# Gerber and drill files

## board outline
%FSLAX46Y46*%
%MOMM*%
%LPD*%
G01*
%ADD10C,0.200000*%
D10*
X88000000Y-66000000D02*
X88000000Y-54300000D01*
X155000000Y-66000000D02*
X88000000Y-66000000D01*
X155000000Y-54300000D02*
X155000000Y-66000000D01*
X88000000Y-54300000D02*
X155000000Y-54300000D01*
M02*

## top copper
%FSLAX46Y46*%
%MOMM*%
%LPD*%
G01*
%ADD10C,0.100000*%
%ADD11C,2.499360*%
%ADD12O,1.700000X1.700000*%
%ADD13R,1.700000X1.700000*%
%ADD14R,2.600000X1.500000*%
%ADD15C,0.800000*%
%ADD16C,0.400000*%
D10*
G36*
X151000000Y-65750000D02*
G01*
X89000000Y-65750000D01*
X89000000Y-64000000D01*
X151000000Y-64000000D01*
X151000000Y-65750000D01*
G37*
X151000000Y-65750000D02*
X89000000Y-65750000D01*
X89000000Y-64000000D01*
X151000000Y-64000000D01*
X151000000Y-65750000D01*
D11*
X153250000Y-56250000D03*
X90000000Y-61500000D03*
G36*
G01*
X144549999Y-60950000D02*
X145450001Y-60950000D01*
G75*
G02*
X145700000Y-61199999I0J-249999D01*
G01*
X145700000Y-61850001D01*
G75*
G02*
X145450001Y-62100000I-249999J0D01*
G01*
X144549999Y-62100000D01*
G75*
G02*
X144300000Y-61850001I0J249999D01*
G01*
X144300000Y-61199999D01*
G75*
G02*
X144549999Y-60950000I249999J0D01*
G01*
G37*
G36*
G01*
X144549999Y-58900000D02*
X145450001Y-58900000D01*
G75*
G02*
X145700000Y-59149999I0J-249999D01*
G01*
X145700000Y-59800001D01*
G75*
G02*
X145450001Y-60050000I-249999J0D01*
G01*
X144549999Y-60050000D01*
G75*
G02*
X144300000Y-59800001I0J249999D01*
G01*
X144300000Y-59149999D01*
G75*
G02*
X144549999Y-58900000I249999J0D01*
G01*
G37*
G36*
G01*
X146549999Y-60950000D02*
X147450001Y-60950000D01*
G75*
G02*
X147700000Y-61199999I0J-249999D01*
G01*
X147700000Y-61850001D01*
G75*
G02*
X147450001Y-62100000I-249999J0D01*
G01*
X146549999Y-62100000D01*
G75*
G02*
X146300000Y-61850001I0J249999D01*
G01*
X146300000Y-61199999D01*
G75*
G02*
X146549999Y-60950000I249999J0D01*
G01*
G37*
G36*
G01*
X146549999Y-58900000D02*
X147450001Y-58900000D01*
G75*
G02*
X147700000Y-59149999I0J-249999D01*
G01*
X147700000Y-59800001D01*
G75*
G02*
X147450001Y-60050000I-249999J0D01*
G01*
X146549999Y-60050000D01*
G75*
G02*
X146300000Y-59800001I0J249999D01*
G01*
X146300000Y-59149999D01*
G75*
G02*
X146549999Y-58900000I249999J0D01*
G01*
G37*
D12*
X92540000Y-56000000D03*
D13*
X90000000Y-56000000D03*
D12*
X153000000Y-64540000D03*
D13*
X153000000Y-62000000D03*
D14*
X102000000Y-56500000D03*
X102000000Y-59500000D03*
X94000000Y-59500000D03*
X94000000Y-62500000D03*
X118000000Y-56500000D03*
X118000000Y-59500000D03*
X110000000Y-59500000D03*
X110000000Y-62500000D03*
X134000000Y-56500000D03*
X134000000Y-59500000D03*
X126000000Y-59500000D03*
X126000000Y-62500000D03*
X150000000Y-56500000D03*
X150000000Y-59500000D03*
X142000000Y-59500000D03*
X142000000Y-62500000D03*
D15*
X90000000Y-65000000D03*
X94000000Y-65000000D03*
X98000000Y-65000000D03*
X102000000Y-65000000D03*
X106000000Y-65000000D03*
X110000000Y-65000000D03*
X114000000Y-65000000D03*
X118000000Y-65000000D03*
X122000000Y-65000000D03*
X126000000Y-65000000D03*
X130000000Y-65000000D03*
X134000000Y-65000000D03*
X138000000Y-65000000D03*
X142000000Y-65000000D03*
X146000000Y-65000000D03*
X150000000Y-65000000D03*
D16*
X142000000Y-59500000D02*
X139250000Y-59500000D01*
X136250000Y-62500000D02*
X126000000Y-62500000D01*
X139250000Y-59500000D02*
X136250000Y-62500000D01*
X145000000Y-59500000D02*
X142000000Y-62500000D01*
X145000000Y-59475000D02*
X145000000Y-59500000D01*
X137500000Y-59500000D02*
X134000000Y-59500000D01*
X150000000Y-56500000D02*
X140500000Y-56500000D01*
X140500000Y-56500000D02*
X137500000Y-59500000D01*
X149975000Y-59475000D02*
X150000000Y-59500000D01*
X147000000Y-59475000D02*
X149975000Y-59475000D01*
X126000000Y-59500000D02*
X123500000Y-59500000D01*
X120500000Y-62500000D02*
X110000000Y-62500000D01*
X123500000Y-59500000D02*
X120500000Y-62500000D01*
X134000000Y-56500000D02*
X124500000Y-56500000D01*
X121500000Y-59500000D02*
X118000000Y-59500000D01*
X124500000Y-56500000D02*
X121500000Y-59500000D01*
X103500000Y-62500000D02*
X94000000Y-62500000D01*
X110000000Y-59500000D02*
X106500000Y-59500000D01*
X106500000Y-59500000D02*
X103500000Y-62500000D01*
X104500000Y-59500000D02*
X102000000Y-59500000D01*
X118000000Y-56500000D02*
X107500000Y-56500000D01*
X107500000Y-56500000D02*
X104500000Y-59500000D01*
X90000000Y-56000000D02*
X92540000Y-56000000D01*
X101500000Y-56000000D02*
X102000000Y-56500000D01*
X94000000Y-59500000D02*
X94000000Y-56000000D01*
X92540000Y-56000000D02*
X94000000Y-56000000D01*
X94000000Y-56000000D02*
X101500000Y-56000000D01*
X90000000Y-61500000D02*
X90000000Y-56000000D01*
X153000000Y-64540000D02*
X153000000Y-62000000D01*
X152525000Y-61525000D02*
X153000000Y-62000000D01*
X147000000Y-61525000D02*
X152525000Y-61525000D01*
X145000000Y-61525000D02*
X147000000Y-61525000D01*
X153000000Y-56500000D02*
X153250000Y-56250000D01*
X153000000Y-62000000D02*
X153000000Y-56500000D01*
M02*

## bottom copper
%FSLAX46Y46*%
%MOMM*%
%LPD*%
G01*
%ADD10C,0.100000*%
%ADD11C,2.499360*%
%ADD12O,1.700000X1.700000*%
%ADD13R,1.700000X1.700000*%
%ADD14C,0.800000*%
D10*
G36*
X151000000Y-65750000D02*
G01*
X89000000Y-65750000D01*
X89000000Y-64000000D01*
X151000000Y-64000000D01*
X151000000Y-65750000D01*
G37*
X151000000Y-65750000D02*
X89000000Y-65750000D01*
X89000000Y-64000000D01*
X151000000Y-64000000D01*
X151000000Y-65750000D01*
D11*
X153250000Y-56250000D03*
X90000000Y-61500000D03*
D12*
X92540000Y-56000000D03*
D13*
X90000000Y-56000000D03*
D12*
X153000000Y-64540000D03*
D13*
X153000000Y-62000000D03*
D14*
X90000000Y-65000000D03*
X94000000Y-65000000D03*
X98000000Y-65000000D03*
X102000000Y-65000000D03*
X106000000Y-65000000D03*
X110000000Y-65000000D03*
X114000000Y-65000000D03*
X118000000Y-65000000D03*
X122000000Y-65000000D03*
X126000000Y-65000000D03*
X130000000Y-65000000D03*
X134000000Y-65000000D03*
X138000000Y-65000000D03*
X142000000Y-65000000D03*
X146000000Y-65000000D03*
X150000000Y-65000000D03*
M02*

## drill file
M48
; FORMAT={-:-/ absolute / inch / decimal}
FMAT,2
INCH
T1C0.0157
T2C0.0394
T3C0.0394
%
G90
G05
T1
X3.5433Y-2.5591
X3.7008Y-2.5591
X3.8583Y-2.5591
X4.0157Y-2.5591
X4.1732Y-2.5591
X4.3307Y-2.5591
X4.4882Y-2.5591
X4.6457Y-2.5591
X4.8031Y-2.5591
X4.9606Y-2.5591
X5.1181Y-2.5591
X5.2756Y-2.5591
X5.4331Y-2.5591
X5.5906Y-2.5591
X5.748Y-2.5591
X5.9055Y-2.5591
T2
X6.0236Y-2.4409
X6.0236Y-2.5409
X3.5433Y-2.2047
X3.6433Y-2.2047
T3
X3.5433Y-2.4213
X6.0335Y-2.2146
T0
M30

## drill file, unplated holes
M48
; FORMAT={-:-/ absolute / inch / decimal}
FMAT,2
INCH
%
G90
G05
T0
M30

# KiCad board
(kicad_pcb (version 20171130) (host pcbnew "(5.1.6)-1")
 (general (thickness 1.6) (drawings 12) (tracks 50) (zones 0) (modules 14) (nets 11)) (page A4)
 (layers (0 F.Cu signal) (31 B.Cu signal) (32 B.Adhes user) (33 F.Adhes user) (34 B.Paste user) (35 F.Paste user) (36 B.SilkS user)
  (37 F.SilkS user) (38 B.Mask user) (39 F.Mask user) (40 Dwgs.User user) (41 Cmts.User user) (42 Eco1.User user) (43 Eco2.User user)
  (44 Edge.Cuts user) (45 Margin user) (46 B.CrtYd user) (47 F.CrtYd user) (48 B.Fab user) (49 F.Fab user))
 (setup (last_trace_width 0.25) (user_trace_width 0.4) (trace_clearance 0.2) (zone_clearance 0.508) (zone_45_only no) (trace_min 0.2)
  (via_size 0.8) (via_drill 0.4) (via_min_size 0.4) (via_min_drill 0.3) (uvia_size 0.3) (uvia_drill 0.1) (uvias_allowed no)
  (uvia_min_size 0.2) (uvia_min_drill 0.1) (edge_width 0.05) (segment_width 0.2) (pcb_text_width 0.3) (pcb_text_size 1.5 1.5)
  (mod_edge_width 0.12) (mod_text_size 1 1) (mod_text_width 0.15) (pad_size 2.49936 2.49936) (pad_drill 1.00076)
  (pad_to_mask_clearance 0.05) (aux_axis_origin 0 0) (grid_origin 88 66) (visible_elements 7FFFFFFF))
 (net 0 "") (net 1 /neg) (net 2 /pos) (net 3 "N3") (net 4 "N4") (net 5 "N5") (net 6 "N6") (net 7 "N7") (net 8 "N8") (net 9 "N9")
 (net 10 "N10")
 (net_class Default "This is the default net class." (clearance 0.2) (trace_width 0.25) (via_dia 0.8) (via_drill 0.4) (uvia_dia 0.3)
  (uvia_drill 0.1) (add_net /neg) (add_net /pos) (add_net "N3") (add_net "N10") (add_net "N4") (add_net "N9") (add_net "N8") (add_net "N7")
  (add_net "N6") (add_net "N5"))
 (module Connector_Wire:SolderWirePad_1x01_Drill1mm (layer F.Cu) (at 153.25 56.25)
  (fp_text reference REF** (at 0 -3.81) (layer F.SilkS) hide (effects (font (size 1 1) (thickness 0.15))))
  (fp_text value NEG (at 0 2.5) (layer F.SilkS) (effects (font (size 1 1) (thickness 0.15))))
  (pad 1 thru_hole circle (at 0 0) (size 2.49936 2.49936) (drill 1.00076) (layers *.Cu *.Mask) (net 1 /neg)))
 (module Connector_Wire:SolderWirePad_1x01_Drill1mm (layer F.Cu) (at 90 61.5)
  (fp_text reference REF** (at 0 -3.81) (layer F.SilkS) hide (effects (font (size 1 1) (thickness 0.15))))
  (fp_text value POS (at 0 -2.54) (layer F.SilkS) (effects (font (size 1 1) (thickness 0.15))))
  (pad 1 thru_hole circle (at 0 0) (size 2.49936 2.49936) (drill 1.00076) (layers *.Cu *.Mask) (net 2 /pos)))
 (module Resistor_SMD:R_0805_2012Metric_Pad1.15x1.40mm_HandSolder (layer F.Cu) (at 145 60.5 270)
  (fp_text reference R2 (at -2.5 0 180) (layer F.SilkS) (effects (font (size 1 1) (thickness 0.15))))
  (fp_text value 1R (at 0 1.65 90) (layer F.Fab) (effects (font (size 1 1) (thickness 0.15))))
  (pad 2 smd roundrect (at 1.025 0 270) (size 1.15 1.4) (layers F.Cu F.Paste F.Mask) (roundrect_rratio 0.217391) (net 1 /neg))
  (pad 1 smd roundrect (at -1.025 0 270) (size 1.15 1.4) (layers F.Cu F.Paste F.Mask) (roundrect_rratio 0.217391) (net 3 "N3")))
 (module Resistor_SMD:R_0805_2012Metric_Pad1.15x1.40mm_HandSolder (layer F.Cu) (at 147 60.5 270)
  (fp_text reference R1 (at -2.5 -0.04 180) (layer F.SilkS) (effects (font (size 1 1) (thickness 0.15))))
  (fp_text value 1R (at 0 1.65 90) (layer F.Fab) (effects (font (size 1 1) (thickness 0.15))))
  (pad 2 smd roundrect (at 1.025 0 270) (size 1.15 1.4) (layers F.Cu F.Paste F.Mask) (roundrect_rratio 0.217391) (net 1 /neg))
  (pad 1 smd roundrect (at -1.025 0 270) (size 1.15 1.4) (layers F.Cu F.Paste F.Mask) (roundrect_rratio 0.217391) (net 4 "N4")))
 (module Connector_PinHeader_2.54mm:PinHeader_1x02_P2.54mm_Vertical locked (layer B.Cu) (at 90 56 270)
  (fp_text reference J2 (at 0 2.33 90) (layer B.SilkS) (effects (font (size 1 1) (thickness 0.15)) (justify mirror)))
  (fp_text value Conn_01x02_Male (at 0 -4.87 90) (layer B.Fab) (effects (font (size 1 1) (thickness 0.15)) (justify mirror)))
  (pad 2 thru_hole oval (at 0 -2.54 270) (size 1.7 1.7) (drill 1) (layers *.Cu *.Mask) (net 2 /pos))
  (pad 1 thru_hole rect (at 0 0 270) (size 1.7 1.7) (drill 1) (layers *.Cu *.Mask) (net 2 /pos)))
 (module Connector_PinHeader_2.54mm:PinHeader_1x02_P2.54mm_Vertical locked (layer B.Cu) (at 153 62 180)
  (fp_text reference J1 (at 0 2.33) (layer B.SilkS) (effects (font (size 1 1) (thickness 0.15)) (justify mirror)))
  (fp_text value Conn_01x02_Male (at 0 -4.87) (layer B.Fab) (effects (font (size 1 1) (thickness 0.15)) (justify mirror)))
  (pad 2 thru_hole oval (at 0 -2.54 180) (size 1.7 1.7) (drill 1) (layers *.Cu *.Mask) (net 1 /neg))
  (pad 1 thru_hole rect (at 0 0 180) (size 1.7 1.7) (drill 1) (layers *.Cu *.Mask) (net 1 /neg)))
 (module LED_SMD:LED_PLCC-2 (layer F.Cu) (at 102 58 90)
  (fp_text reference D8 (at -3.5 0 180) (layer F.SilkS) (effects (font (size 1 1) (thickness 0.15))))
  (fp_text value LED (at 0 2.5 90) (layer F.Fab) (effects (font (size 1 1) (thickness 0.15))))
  (pad 2 smd rect (at 1.5 0 90) (size 1.5 2.6) (layers F.Cu F.Paste F.Mask) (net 2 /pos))
  (pad 1 smd rect (at -1.5 0 90) (size 1.5 2.6) (layers F.Cu F.Paste F.Mask) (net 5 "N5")))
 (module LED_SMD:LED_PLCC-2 (layer F.Cu) (at 94 61 90)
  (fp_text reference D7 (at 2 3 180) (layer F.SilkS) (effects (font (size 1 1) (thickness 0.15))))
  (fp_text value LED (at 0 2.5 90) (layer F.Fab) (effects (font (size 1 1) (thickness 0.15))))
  (pad 2 smd rect (at 1.5 0 90) (size 1.5 2.6) (layers F.Cu F.Paste F.Mask) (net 2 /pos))
  (pad 1 smd rect (at -1.5 0 90) (size 1.5 2.6) (layers F.Cu F.Paste F.Mask) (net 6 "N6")))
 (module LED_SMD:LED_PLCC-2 (layer F.Cu) (at 118 58 90)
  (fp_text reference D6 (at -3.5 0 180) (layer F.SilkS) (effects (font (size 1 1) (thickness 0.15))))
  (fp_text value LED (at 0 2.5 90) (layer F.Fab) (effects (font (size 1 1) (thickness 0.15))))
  (pad 2 smd rect (at 1.5 0 90) (size 1.5 2.6) (layers F.Cu F.Paste F.Mask) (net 5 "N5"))
  (pad 1 smd rect (at -1.5 0 90) (size 1.5 2.6) (layers F.Cu F.Paste F.Mask) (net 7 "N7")))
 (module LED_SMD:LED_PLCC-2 (layer F.Cu) (at 110 61 90)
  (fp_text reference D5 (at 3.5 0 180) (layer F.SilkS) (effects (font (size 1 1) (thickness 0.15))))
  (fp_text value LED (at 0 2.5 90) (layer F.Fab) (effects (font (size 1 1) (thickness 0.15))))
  (pad 2 smd rect (at 1.5 0 90) (size 1.5 2.6) (layers F.Cu F.Paste F.Mask) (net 6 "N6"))
  (pad 1 smd rect (at -1.5 0 90) (size 1.5 2.6) (layers F.Cu F.Paste F.Mask) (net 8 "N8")))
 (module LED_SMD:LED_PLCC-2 (layer F.Cu) (at 134 58 90)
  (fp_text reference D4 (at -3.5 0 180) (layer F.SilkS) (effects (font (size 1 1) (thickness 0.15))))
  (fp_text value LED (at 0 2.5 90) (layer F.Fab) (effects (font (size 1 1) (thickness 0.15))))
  (pad 2 smd rect (at 1.5 0 90) (size 1.5 2.6) (layers F.Cu F.Paste F.Mask) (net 7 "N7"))
  (pad 1 smd rect (at -1.5 0 90) (size 1.5 2.6) (layers F.Cu F.Paste F.Mask) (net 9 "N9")))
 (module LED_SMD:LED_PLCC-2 (layer F.Cu) (at 126 61 90)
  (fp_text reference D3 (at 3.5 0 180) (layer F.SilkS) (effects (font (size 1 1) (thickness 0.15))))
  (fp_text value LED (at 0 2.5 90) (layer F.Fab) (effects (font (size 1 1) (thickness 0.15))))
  (pad 2 smd rect (at 1.5 0 90) (size 1.5 2.6) (layers F.Cu F.Paste F.Mask) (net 8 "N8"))
  (pad 1 smd rect (at -1.5 0 90) (size 1.5 2.6) (layers F.Cu F.Paste F.Mask) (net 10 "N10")))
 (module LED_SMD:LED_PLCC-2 (layer F.Cu) (at 150 58 90)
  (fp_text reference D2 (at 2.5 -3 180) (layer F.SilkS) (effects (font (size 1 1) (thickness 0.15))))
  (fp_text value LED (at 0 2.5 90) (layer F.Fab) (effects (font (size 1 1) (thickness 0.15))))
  (pad 2 smd rect (at 1.5 0 90) (size 1.5 2.6) (layers F.Cu F.Paste F.Mask) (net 9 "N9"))
  (pad 1 smd rect (at -1.5 0 90) (size 1.5 2.6) (layers F.Cu F.Paste F.Mask) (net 4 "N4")))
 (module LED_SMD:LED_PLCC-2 (layer F.Cu) (at 142 61 90)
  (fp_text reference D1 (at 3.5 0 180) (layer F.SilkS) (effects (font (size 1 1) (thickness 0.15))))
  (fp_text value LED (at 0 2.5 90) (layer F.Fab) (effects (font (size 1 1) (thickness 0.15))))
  (pad 2 smd rect (at 1.5 0 90) (size 1.5 2.6) (layers F.Cu F.Paste F.Mask) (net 10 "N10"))
  (pad 1 smd rect (at -1.5 0 90) (size 1.5 2.6) (layers F.Cu F.Paste F.Mask) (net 3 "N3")))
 (gr_poly (pts (xy 151 65.75) (xy 89 65.75) (xy 89 64) (xy 151 64)) (layer B.Cu) (width 0.1))
 (gr_poly (pts (xy 151 65.75) (xy 89 65.75) (xy 89 64) (xy 151 64)) (layer F.Cu) (width 0.1))
 (gr_line (start 88 66) (end 88 54.3) (layer Edge.Cuts) (width 0.2))
 (gr_line (start 155 66) (end 88 66) (layer Edge.Cuts) (width 0.2))
 (gr_line (start 155 54.3) (end 155 66) (layer Edge.Cuts) (width 0.2))
 (gr_line (start 88 54.3) (end 155 54.3) (layer Edge.Cuts) (width 0.2))
 (via (at 90 65) (size 0.8) (drill 0.4) (layers F.Cu B.Cu) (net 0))
 (via (at 94 65) (size 0.8) (drill 0.4) (layers F.Cu B.Cu) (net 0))
 (via (at 98 65) (size 0.8) (drill 0.4) (layers F.Cu B.Cu) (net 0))
 (via (at 102 65) (size 0.8) (drill 0.4) (layers F.Cu B.Cu) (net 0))
 (via (at 106 65) (size 0.8) (drill 0.4) (layers F.Cu B.Cu) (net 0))
 (via (at 110 65) (size 0.8) (drill 0.4) (layers F.Cu B.Cu) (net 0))
 (via (at 114 65) (size 0.8) (drill 0.4) (layers F.Cu B.Cu) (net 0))
 (via (at 118 65) (size 0.8) (drill 0.4) (layers F.Cu B.Cu) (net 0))
 (via (at 122 65) (size 0.8) (drill 0.4) (layers F.Cu B.Cu) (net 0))
 (via (at 126 65) (size 0.8) (drill 0.4) (layers F.Cu B.Cu) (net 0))
 (via (at 130 65) (size 0.8) (drill 0.4) (layers F.Cu B.Cu) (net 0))
 (via (at 134 65) (size 0.8) (drill 0.4) (layers F.Cu B.Cu) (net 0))
 (via (at 138 65) (size 0.8) (drill 0.4) (layers F.Cu B.Cu) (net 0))
 (via (at 142 65) (size 0.8) (drill 0.4) (layers F.Cu B.Cu) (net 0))
 (via (at 146 65) (size 0.8) (drill 0.4) (layers F.Cu B.Cu) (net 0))
 (via (at 150 65) (size 0.8) (drill 0.4) (layers F.Cu B.Cu) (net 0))
 (segment (start 142 59.5) (end 139.25 59.5) (width 0.4) (layer F.Cu) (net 10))
 (segment (start 136.25 62.5) (end 126 62.5) (width 0.4) (layer F.Cu) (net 10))
 (segment (start 139.25 59.5) (end 136.25 62.5) (width 0.4) (layer F.Cu) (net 10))
 (segment (start 145 59.5) (end 142 62.5) (width 0.4) (layer F.Cu) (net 3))
 (segment (start 145 59.475) (end 145 59.5) (width 0.4) (layer F.Cu) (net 3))
 (segment (start 137.5 59.5) (end 134 59.5) (width 0.4) (layer F.Cu) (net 9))
 (segment (start 150 56.5) (end 140.5 56.5) (width 0.4) (layer F.Cu) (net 9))
 (segment (start 140.5 56.5) (end 137.5 59.5) (width 0.4) (layer F.Cu) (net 9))
 (segment (start 149.975 59.475) (end 150 59.5) (width 0.4) (layer F.Cu) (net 4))
 (segment (start 147 59.475) (end 149.975 59.475) (width 0.4) (layer F.Cu) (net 4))
 (segment (start 126 59.5) (end 123.5 59.5) (width 0.4) (layer F.Cu) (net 8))
 (segment (start 120.5 62.5) (end 110 62.5) (width 0.4) (layer F.Cu) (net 8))
 (segment (start 123.5 59.5) (end 120.5 62.5) (width 0.4) (layer F.Cu) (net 8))
 (segment (start 134 56.5) (end 124.5 56.5) (width 0.4) (layer F.Cu) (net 7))
 (segment (start 121.5 59.5) (end 118 59.5) (width 0.4) (layer F.Cu) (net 7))
 (segment (start 124.5 56.5) (end 121.5 59.5) (width 0.4) (layer F.Cu) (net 7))
 (segment (start 103.5 62.5) (end 94 62.5) (width 0.4) (layer F.Cu) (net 6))
 (segment (start 110 59.5) (end 106.5 59.5) (width 0.4) (layer F.Cu) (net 6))
 (segment (start 106.5 59.5) (end 103.5 62.5) (width 0.4) (layer F.Cu) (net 6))
 (segment (start 104.5 59.5) (end 102 59.5) (width 0.4) (layer F.Cu) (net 5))
 (segment (start 118 56.5) (end 107.5 56.5) (width 0.4) (layer F.Cu) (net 5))
 (segment (start 107.5 56.5) (end 104.5 59.5) (width 0.4) (layer F.Cu) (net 5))
 (segment (start 90 56) (end 92.54 56) (width 0.4) (layer F.Cu) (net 2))
 (segment (start 101.5 56) (end 102 56.5) (width 0.4) (layer F.Cu) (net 2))
 (segment (start 94 59.5) (end 94 56) (width 0.4) (layer F.Cu) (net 2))
 (segment (start 92.54 56) (end 94 56) (width 0.4) (layer F.Cu) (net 2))
 (segment (start 94 56) (end 101.5 56) (width 0.4) (layer F.Cu) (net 2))
 (segment (start 90 61.5) (end 90 56) (width 0.4) (layer F.Cu) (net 2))
 (segment (start 153 64.54) (end 153 62) (width 0.4) (layer F.Cu) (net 1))
 (segment (start 152.525 61.525) (end 153 62) (width 0.4) (layer F.Cu) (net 1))
 (segment (start 147 61.525) (end 152.525 61.525) (width 0.4) (layer F.Cu) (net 1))
 (segment (start 145 61.525) (end 147 61.525) (width 0.4) (layer F.Cu) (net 1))
 (segment (start 153 56.5) (end 153.25 56.25) (width 0.4) (layer F.Cu) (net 1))
 (segment (start 153 62) (end 153 56.5) (width 0.4) (layer F.Cu) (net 1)))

